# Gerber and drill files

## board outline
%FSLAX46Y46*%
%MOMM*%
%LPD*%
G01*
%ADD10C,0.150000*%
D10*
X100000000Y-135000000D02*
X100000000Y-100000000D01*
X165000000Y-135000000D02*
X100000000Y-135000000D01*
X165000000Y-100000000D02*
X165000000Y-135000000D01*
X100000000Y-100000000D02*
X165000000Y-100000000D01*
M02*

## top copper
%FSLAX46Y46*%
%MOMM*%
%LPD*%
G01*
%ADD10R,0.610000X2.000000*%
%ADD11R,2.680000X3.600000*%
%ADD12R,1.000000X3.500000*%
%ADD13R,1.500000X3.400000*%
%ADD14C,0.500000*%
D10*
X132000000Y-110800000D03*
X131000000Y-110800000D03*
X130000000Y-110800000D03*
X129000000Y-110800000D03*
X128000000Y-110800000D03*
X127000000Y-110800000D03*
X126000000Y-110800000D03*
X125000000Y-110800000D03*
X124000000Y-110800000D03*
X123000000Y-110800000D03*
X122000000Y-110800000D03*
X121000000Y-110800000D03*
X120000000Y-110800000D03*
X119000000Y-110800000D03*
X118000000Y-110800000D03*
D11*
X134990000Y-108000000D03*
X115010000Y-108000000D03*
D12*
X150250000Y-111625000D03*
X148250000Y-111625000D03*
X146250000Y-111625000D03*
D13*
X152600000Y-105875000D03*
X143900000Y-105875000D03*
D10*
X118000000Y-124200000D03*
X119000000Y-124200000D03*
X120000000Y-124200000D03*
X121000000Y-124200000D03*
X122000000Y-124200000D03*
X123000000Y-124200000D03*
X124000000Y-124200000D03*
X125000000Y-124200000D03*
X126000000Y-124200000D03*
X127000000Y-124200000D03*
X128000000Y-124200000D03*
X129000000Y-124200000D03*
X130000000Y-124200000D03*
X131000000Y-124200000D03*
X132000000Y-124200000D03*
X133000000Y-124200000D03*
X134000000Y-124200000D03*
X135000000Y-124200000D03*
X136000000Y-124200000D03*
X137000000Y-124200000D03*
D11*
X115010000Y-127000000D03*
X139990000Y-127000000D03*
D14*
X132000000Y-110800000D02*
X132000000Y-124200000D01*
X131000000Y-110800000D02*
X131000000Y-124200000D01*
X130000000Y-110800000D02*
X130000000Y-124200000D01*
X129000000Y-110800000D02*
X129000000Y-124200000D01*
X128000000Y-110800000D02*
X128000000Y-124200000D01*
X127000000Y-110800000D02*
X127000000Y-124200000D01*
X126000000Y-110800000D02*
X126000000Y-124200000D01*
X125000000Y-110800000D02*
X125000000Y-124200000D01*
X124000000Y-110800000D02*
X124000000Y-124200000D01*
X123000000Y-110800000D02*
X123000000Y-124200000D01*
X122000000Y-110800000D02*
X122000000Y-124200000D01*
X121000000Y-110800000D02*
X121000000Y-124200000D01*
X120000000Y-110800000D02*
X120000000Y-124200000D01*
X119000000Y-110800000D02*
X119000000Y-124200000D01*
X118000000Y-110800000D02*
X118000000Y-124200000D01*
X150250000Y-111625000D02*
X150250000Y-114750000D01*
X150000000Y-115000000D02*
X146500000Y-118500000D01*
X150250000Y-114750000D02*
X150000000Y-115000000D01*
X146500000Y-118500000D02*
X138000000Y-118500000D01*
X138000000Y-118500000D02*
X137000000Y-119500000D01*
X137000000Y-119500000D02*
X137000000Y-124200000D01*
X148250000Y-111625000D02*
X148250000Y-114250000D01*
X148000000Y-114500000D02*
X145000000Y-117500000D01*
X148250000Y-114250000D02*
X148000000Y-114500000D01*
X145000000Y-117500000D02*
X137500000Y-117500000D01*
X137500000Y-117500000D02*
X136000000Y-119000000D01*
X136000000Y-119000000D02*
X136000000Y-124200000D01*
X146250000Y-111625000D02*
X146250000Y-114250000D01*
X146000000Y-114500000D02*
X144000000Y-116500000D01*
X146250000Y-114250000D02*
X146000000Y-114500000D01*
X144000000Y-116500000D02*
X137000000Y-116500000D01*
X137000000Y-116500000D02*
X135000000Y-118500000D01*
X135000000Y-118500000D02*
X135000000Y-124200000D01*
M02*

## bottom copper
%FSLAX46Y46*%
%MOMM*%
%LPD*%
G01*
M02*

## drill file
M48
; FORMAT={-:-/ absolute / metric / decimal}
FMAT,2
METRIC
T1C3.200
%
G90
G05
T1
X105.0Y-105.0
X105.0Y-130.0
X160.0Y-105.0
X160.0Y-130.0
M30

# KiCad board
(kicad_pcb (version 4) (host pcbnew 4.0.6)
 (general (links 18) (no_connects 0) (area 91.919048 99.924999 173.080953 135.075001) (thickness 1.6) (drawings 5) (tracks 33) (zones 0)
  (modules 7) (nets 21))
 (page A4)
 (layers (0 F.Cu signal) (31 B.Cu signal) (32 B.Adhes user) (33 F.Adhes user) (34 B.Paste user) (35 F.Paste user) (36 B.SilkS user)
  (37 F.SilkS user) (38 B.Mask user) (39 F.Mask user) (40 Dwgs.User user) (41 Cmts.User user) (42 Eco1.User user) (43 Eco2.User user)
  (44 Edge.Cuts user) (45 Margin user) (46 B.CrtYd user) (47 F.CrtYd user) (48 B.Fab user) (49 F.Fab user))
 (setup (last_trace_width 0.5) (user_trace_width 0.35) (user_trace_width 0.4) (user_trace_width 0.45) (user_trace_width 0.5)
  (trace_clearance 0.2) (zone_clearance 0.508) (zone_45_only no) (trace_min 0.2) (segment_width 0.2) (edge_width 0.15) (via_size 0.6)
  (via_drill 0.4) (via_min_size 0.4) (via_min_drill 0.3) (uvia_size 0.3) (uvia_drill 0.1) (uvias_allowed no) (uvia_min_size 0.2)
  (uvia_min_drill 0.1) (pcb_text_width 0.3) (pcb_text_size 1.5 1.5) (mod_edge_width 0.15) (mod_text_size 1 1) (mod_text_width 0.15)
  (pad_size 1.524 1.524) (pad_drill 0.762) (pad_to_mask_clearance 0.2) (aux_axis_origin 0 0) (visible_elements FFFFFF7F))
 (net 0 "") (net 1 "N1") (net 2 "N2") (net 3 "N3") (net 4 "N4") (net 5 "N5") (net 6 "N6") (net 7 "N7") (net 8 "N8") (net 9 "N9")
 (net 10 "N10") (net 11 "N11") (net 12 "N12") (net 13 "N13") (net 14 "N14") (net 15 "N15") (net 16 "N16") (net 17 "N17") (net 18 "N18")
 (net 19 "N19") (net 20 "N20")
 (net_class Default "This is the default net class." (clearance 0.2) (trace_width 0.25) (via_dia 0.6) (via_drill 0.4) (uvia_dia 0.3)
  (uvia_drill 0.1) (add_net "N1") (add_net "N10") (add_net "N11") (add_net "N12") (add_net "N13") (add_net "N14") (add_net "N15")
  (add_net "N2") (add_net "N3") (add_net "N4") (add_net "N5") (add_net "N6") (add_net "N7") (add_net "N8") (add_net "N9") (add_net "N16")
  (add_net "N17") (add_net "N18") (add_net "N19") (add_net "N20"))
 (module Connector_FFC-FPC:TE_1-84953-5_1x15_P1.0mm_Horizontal (layer F.Cu) (at 125 109 180)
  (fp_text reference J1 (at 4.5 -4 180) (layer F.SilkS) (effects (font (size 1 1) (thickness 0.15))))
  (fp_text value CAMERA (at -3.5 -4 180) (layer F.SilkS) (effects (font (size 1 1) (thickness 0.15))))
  (pad 1 smd rect (at -7 -1.8 180) (size 0.61 2) (layers F.Cu F.Paste F.Mask) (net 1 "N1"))
  (pad 2 smd rect (at -6 -1.8 180) (size 0.61 2) (layers F.Cu F.Paste F.Mask) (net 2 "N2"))
  (pad 3 smd rect (at -5 -1.8 180) (size 0.61 2) (layers F.Cu F.Paste F.Mask) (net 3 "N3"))
  (pad 4 smd rect (at -4 -1.8 180) (size 0.61 2) (layers F.Cu F.Paste F.Mask) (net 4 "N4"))
  (pad 5 smd rect (at -3 -1.8 180) (size 0.61 2) (layers F.Cu F.Paste F.Mask) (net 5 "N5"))
  (pad 6 smd rect (at -2 -1.8 180) (size 0.61 2) (layers F.Cu F.Paste F.Mask) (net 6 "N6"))
  (pad 7 smd rect (at -1 -1.8 180) (size 0.61 2) (layers F.Cu F.Paste F.Mask) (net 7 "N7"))
  (pad 8 smd rect (at 0 -1.8 180) (size 0.61 2) (layers F.Cu F.Paste F.Mask) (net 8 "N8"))
  (pad 9 smd rect (at 1 -1.8 180) (size 0.61 2) (layers F.Cu F.Paste F.Mask) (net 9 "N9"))
  (pad 10 smd rect (at 2 -1.8 180) (size 0.61 2) (layers F.Cu F.Paste F.Mask) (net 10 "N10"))
  (pad 11 smd rect (at 3 -1.8 180) (size 0.61 2) (layers F.Cu F.Paste F.Mask) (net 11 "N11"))
  (pad 12 smd rect (at 4 -1.8 180) (size 0.61 2) (layers F.Cu F.Paste F.Mask) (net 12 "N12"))
  (pad 13 smd rect (at 5 -1.8 180) (size 0.61 2) (layers F.Cu F.Paste F.Mask) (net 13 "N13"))
  (pad 14 smd rect (at 6 -1.8 180) (size 0.61 2) (layers F.Cu F.Paste F.Mask) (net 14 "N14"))
  (pad 15 smd rect (at 7 -1.8 180) (size 0.61 2) (layers F.Cu F.Paste F.Mask) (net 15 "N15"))
  (pad "" smd rect (at -9.99 1 180) (size 2.68 3.6) (layers F.Cu F.Paste F.Mask))
  (pad "" smd rect (at 9.99 1 180) (size 2.68 3.6) (layers F.Cu F.Paste F.Mask)))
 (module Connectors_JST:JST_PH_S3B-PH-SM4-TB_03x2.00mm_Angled (layer F.Cu) (at 148.25 108.75 180)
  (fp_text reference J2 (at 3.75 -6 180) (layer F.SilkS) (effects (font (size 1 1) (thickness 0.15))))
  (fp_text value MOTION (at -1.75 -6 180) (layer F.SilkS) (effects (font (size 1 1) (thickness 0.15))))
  (pad 1 smd rect (at -2 -2.875 180) (size 1 3.5) (layers F.Cu F.Paste F.Mask) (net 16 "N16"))
  (pad 2 smd rect (at 0 -2.875 180) (size 1 3.5) (layers F.Cu F.Paste F.Mask) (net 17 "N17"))
  (pad 3 smd rect (at 2 -2.875 180) (size 1 3.5) (layers F.Cu F.Paste F.Mask) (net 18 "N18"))
  (pad "" smd rect (at -4.35 2.875 180) (size 1.5 3.4) (layers F.Cu F.Paste F.Mask))
  (pad "" smd rect (at 4.35 2.875 180) (size 1.5 3.4) (layers F.Cu F.Paste F.Mask)))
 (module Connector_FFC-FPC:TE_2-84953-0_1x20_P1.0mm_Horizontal (layer F.Cu) (at 127.5 126)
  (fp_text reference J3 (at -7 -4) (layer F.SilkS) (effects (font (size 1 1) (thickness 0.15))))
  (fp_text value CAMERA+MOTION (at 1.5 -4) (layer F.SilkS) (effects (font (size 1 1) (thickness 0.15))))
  (pad 1 smd rect (at -9.5 -1.8) (size 0.61 2) (layers F.Cu F.Paste F.Mask) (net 15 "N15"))
  (pad 2 smd rect (at -8.5 -1.8) (size 0.61 2) (layers F.Cu F.Paste F.Mask) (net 14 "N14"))
  (pad 3 smd rect (at -7.5 -1.8) (size 0.61 2) (layers F.Cu F.Paste F.Mask) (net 13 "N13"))
  (pad 4 smd rect (at -6.5 -1.8) (size 0.61 2) (layers F.Cu F.Paste F.Mask) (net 12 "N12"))
  (pad 5 smd rect (at -5.5 -1.8) (size 0.61 2) (layers F.Cu F.Paste F.Mask) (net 11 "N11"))
  (pad 6 smd rect (at -4.5 -1.8) (size 0.61 2) (layers F.Cu F.Paste F.Mask) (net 10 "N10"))
  (pad 7 smd rect (at -3.5 -1.8) (size 0.61 2) (layers F.Cu F.Paste F.Mask) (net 9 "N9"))
  (pad 8 smd rect (at -2.5 -1.8) (size 0.61 2) (layers F.Cu F.Paste F.Mask) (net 8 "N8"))
  (pad 9 smd rect (at -1.5 -1.8) (size 0.61 2) (layers F.Cu F.Paste F.Mask) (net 7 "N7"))
  (pad 10 smd rect (at -0.5 -1.8) (size 0.61 2) (layers F.Cu F.Paste F.Mask) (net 6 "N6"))
  (pad 11 smd rect (at 0.5 -1.8) (size 0.61 2) (layers F.Cu F.Paste F.Mask) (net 5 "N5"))
  (pad 12 smd rect (at 1.5 -1.8) (size 0.61 2) (layers F.Cu F.Paste F.Mask) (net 4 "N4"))
  (pad 13 smd rect (at 2.5 -1.8) (size 0.61 2) (layers F.Cu F.Paste F.Mask) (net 3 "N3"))
  (pad 14 smd rect (at 3.5 -1.8) (size 0.61 2) (layers F.Cu F.Paste F.Mask) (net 2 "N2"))
  (pad 15 smd rect (at 4.5 -1.8) (size 0.61 2) (layers F.Cu F.Paste F.Mask) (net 1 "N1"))
  (pad 16 smd rect (at 5.5 -1.8) (size 0.61 2) (layers F.Cu F.Paste F.Mask) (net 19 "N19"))
  (pad 17 smd rect (at 6.5 -1.8) (size 0.61 2) (layers F.Cu F.Paste F.Mask) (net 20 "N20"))
  (pad 18 smd rect (at 7.5 -1.8) (size 0.61 2) (layers F.Cu F.Paste F.Mask) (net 18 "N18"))
  (pad 19 smd rect (at 8.5 -1.8) (size 0.61 2) (layers F.Cu F.Paste F.Mask) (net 17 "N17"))
  (pad 20 smd rect (at 9.5 -1.8) (size 0.61 2) (layers F.Cu F.Paste F.Mask) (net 16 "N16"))
  (pad "" smd rect (at -12.49 1) (size 2.68 3.6) (layers F.Cu F.Paste F.Mask))
  (pad "" smd rect (at 12.49 1) (size 2.68 3.6) (layers F.Cu F.Paste F.Mask)))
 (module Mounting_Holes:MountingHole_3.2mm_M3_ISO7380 (layer F.Cu) (at 105 105)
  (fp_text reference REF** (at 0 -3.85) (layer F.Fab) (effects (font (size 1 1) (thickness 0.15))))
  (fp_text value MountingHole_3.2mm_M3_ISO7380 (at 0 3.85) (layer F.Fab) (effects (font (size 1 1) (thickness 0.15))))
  (pad 1 np_thru_hole circle (at 0 0) (size 3.2 3.2) (drill 3.2) (layers *.Cu *.Mask)))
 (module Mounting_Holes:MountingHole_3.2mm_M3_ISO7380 (layer F.Cu) (at 105 130)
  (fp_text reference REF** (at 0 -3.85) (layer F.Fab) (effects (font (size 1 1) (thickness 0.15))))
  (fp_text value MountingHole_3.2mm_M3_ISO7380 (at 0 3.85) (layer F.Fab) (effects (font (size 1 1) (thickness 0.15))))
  (pad 1 np_thru_hole circle (at 0 0) (size 3.2 3.2) (drill 3.2) (layers *.Cu *.Mask)))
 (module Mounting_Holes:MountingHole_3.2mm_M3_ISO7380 (layer F.Cu) (at 160 130)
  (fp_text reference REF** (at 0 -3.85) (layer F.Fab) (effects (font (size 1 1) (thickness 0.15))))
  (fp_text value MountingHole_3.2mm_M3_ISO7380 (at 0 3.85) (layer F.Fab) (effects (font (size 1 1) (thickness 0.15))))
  (pad 1 np_thru_hole circle (at 0 0) (size 3.2 3.2) (drill 3.2) (layers *.Cu *.Mask)))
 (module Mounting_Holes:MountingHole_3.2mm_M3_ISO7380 (layer F.Cu) (at 160 105)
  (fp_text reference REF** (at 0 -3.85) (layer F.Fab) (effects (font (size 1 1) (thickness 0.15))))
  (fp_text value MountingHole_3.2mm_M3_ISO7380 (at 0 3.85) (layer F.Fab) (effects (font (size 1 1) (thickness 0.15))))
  (pad 1 np_thru_hole circle (at 0 0) (size 3.2 3.2) (drill 3.2) (layers *.Cu *.Mask)))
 (gr_line (start 100 135) (end 100 100) (angle 90) (layer Edge.Cuts) (width 0.15))
 (gr_line (start 165 135) (end 100 135) (angle 90) (layer Edge.Cuts) (width 0.15))
 (gr_line (start 165 100) (end 165 135) (angle 90) (layer Edge.Cuts) (width 0.15))
 (gr_line (start 100 100) (end 165 100) (angle 90) (layer Edge.Cuts) (width 0.15))
 (segment (start 132 110.8) (end 132 124.2) (width 0.5) (layer F.Cu) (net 1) (status 20))
 (segment (start 131 110.8) (end 131 124.2) (width 0.5) (layer F.Cu) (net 2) (status 20))
 (segment (start 130 110.8) (end 130 124.2) (width 0.5) (layer F.Cu) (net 3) (status 20))
 (segment (start 129 110.8) (end 129 124.2) (width 0.5) (layer F.Cu) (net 4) (status 20))
 (segment (start 128 110.8) (end 128 124.2) (width 0.5) (layer F.Cu) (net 5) (status 20))
 (segment (start 127 110.8) (end 127 124.2) (width 0.5) (layer F.Cu) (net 6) (status 20))
 (segment (start 126 110.8) (end 126 124.2) (width 0.5) (layer F.Cu) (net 7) (status 20))
 (segment (start 125 110.8) (end 125 124.2) (width 0.5) (layer F.Cu) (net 8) (status 20))
 (segment (start 124 110.8) (end 124 124.2) (width 0.5) (layer F.Cu) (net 9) (status 20))
 (segment (start 123 110.8) (end 123 124.2) (width 0.5) (layer F.Cu) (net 10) (status 20))
 (segment (start 122 110.8) (end 122 124.2) (width 0.5) (layer F.Cu) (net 11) (status 20))
 (segment (start 121 110.8) (end 121 124.2) (width 0.5) (layer F.Cu) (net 12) (status 20))
 (segment (start 120 110.8) (end 120 124.2) (width 0.5) (layer F.Cu) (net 13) (status 20))
 (segment (start 119 110.8) (end 119 124.2) (width 0.5) (layer F.Cu) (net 14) (status 20))
 (segment (start 118 110.8) (end 118 124.2) (width 0.5) (layer F.Cu) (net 15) (status 20))
 (segment (start 150.25 111.625) (end 150.25 114.75) (width 0.5) (layer F.Cu) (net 16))
 (segment (start 150 115) (end 146.5 118.5) (width 0.5) (layer F.Cu) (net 16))
 (segment (start 150.25 114.75) (end 150 115) (width 0.5) (layer F.Cu) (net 16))
 (segment (start 146.5 118.5) (end 138 118.5) (width 0.5) (layer F.Cu) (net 16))
 (segment (start 138 118.5) (end 137 119.5) (width 0.5) (layer F.Cu) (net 16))
 (segment (start 137 119.5) (end 137 124.2) (width 0.5) (layer F.Cu) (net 16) (status 20))
 (segment (start 148.25 111.625) (end 148.25 114.25) (width 0.5) (layer F.Cu) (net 17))
 (segment (start 148 114.5) (end 145 117.5) (width 0.5) (layer F.Cu) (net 17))
 (segment (start 148.25 114.25) (end 148 114.5) (width 0.5) (layer F.Cu) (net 17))
 (segment (start 145 117.5) (end 137.5 117.5) (width 0.5) (layer F.Cu) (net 17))
 (segment (start 137.5 117.5) (end 136 119) (width 0.5) (layer F.Cu) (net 17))
 (segment (start 136 119) (end 136 124.2) (width 0.5) (layer F.Cu) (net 17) (status 20))
 (segment (start 146.25 111.625) (end 146.25 114.25) (width 0.5) (layer F.Cu) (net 18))
 (segment (start 146 114.5) (end 144 116.5) (width 0.5) (layer F.Cu) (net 18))
 (segment (start 146.25 114.25) (end 146 114.5) (width 0.5) (layer F.Cu) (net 18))
 (segment (start 144 116.5) (end 137 116.5) (width 0.5) (layer F.Cu) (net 18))
 (segment (start 137 116.5) (end 135 118.5) (width 0.5) (layer F.Cu) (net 18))
 (segment (start 135 118.5) (end 135 124.2) (width 0.5) (layer F.Cu) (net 18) (status 20)))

